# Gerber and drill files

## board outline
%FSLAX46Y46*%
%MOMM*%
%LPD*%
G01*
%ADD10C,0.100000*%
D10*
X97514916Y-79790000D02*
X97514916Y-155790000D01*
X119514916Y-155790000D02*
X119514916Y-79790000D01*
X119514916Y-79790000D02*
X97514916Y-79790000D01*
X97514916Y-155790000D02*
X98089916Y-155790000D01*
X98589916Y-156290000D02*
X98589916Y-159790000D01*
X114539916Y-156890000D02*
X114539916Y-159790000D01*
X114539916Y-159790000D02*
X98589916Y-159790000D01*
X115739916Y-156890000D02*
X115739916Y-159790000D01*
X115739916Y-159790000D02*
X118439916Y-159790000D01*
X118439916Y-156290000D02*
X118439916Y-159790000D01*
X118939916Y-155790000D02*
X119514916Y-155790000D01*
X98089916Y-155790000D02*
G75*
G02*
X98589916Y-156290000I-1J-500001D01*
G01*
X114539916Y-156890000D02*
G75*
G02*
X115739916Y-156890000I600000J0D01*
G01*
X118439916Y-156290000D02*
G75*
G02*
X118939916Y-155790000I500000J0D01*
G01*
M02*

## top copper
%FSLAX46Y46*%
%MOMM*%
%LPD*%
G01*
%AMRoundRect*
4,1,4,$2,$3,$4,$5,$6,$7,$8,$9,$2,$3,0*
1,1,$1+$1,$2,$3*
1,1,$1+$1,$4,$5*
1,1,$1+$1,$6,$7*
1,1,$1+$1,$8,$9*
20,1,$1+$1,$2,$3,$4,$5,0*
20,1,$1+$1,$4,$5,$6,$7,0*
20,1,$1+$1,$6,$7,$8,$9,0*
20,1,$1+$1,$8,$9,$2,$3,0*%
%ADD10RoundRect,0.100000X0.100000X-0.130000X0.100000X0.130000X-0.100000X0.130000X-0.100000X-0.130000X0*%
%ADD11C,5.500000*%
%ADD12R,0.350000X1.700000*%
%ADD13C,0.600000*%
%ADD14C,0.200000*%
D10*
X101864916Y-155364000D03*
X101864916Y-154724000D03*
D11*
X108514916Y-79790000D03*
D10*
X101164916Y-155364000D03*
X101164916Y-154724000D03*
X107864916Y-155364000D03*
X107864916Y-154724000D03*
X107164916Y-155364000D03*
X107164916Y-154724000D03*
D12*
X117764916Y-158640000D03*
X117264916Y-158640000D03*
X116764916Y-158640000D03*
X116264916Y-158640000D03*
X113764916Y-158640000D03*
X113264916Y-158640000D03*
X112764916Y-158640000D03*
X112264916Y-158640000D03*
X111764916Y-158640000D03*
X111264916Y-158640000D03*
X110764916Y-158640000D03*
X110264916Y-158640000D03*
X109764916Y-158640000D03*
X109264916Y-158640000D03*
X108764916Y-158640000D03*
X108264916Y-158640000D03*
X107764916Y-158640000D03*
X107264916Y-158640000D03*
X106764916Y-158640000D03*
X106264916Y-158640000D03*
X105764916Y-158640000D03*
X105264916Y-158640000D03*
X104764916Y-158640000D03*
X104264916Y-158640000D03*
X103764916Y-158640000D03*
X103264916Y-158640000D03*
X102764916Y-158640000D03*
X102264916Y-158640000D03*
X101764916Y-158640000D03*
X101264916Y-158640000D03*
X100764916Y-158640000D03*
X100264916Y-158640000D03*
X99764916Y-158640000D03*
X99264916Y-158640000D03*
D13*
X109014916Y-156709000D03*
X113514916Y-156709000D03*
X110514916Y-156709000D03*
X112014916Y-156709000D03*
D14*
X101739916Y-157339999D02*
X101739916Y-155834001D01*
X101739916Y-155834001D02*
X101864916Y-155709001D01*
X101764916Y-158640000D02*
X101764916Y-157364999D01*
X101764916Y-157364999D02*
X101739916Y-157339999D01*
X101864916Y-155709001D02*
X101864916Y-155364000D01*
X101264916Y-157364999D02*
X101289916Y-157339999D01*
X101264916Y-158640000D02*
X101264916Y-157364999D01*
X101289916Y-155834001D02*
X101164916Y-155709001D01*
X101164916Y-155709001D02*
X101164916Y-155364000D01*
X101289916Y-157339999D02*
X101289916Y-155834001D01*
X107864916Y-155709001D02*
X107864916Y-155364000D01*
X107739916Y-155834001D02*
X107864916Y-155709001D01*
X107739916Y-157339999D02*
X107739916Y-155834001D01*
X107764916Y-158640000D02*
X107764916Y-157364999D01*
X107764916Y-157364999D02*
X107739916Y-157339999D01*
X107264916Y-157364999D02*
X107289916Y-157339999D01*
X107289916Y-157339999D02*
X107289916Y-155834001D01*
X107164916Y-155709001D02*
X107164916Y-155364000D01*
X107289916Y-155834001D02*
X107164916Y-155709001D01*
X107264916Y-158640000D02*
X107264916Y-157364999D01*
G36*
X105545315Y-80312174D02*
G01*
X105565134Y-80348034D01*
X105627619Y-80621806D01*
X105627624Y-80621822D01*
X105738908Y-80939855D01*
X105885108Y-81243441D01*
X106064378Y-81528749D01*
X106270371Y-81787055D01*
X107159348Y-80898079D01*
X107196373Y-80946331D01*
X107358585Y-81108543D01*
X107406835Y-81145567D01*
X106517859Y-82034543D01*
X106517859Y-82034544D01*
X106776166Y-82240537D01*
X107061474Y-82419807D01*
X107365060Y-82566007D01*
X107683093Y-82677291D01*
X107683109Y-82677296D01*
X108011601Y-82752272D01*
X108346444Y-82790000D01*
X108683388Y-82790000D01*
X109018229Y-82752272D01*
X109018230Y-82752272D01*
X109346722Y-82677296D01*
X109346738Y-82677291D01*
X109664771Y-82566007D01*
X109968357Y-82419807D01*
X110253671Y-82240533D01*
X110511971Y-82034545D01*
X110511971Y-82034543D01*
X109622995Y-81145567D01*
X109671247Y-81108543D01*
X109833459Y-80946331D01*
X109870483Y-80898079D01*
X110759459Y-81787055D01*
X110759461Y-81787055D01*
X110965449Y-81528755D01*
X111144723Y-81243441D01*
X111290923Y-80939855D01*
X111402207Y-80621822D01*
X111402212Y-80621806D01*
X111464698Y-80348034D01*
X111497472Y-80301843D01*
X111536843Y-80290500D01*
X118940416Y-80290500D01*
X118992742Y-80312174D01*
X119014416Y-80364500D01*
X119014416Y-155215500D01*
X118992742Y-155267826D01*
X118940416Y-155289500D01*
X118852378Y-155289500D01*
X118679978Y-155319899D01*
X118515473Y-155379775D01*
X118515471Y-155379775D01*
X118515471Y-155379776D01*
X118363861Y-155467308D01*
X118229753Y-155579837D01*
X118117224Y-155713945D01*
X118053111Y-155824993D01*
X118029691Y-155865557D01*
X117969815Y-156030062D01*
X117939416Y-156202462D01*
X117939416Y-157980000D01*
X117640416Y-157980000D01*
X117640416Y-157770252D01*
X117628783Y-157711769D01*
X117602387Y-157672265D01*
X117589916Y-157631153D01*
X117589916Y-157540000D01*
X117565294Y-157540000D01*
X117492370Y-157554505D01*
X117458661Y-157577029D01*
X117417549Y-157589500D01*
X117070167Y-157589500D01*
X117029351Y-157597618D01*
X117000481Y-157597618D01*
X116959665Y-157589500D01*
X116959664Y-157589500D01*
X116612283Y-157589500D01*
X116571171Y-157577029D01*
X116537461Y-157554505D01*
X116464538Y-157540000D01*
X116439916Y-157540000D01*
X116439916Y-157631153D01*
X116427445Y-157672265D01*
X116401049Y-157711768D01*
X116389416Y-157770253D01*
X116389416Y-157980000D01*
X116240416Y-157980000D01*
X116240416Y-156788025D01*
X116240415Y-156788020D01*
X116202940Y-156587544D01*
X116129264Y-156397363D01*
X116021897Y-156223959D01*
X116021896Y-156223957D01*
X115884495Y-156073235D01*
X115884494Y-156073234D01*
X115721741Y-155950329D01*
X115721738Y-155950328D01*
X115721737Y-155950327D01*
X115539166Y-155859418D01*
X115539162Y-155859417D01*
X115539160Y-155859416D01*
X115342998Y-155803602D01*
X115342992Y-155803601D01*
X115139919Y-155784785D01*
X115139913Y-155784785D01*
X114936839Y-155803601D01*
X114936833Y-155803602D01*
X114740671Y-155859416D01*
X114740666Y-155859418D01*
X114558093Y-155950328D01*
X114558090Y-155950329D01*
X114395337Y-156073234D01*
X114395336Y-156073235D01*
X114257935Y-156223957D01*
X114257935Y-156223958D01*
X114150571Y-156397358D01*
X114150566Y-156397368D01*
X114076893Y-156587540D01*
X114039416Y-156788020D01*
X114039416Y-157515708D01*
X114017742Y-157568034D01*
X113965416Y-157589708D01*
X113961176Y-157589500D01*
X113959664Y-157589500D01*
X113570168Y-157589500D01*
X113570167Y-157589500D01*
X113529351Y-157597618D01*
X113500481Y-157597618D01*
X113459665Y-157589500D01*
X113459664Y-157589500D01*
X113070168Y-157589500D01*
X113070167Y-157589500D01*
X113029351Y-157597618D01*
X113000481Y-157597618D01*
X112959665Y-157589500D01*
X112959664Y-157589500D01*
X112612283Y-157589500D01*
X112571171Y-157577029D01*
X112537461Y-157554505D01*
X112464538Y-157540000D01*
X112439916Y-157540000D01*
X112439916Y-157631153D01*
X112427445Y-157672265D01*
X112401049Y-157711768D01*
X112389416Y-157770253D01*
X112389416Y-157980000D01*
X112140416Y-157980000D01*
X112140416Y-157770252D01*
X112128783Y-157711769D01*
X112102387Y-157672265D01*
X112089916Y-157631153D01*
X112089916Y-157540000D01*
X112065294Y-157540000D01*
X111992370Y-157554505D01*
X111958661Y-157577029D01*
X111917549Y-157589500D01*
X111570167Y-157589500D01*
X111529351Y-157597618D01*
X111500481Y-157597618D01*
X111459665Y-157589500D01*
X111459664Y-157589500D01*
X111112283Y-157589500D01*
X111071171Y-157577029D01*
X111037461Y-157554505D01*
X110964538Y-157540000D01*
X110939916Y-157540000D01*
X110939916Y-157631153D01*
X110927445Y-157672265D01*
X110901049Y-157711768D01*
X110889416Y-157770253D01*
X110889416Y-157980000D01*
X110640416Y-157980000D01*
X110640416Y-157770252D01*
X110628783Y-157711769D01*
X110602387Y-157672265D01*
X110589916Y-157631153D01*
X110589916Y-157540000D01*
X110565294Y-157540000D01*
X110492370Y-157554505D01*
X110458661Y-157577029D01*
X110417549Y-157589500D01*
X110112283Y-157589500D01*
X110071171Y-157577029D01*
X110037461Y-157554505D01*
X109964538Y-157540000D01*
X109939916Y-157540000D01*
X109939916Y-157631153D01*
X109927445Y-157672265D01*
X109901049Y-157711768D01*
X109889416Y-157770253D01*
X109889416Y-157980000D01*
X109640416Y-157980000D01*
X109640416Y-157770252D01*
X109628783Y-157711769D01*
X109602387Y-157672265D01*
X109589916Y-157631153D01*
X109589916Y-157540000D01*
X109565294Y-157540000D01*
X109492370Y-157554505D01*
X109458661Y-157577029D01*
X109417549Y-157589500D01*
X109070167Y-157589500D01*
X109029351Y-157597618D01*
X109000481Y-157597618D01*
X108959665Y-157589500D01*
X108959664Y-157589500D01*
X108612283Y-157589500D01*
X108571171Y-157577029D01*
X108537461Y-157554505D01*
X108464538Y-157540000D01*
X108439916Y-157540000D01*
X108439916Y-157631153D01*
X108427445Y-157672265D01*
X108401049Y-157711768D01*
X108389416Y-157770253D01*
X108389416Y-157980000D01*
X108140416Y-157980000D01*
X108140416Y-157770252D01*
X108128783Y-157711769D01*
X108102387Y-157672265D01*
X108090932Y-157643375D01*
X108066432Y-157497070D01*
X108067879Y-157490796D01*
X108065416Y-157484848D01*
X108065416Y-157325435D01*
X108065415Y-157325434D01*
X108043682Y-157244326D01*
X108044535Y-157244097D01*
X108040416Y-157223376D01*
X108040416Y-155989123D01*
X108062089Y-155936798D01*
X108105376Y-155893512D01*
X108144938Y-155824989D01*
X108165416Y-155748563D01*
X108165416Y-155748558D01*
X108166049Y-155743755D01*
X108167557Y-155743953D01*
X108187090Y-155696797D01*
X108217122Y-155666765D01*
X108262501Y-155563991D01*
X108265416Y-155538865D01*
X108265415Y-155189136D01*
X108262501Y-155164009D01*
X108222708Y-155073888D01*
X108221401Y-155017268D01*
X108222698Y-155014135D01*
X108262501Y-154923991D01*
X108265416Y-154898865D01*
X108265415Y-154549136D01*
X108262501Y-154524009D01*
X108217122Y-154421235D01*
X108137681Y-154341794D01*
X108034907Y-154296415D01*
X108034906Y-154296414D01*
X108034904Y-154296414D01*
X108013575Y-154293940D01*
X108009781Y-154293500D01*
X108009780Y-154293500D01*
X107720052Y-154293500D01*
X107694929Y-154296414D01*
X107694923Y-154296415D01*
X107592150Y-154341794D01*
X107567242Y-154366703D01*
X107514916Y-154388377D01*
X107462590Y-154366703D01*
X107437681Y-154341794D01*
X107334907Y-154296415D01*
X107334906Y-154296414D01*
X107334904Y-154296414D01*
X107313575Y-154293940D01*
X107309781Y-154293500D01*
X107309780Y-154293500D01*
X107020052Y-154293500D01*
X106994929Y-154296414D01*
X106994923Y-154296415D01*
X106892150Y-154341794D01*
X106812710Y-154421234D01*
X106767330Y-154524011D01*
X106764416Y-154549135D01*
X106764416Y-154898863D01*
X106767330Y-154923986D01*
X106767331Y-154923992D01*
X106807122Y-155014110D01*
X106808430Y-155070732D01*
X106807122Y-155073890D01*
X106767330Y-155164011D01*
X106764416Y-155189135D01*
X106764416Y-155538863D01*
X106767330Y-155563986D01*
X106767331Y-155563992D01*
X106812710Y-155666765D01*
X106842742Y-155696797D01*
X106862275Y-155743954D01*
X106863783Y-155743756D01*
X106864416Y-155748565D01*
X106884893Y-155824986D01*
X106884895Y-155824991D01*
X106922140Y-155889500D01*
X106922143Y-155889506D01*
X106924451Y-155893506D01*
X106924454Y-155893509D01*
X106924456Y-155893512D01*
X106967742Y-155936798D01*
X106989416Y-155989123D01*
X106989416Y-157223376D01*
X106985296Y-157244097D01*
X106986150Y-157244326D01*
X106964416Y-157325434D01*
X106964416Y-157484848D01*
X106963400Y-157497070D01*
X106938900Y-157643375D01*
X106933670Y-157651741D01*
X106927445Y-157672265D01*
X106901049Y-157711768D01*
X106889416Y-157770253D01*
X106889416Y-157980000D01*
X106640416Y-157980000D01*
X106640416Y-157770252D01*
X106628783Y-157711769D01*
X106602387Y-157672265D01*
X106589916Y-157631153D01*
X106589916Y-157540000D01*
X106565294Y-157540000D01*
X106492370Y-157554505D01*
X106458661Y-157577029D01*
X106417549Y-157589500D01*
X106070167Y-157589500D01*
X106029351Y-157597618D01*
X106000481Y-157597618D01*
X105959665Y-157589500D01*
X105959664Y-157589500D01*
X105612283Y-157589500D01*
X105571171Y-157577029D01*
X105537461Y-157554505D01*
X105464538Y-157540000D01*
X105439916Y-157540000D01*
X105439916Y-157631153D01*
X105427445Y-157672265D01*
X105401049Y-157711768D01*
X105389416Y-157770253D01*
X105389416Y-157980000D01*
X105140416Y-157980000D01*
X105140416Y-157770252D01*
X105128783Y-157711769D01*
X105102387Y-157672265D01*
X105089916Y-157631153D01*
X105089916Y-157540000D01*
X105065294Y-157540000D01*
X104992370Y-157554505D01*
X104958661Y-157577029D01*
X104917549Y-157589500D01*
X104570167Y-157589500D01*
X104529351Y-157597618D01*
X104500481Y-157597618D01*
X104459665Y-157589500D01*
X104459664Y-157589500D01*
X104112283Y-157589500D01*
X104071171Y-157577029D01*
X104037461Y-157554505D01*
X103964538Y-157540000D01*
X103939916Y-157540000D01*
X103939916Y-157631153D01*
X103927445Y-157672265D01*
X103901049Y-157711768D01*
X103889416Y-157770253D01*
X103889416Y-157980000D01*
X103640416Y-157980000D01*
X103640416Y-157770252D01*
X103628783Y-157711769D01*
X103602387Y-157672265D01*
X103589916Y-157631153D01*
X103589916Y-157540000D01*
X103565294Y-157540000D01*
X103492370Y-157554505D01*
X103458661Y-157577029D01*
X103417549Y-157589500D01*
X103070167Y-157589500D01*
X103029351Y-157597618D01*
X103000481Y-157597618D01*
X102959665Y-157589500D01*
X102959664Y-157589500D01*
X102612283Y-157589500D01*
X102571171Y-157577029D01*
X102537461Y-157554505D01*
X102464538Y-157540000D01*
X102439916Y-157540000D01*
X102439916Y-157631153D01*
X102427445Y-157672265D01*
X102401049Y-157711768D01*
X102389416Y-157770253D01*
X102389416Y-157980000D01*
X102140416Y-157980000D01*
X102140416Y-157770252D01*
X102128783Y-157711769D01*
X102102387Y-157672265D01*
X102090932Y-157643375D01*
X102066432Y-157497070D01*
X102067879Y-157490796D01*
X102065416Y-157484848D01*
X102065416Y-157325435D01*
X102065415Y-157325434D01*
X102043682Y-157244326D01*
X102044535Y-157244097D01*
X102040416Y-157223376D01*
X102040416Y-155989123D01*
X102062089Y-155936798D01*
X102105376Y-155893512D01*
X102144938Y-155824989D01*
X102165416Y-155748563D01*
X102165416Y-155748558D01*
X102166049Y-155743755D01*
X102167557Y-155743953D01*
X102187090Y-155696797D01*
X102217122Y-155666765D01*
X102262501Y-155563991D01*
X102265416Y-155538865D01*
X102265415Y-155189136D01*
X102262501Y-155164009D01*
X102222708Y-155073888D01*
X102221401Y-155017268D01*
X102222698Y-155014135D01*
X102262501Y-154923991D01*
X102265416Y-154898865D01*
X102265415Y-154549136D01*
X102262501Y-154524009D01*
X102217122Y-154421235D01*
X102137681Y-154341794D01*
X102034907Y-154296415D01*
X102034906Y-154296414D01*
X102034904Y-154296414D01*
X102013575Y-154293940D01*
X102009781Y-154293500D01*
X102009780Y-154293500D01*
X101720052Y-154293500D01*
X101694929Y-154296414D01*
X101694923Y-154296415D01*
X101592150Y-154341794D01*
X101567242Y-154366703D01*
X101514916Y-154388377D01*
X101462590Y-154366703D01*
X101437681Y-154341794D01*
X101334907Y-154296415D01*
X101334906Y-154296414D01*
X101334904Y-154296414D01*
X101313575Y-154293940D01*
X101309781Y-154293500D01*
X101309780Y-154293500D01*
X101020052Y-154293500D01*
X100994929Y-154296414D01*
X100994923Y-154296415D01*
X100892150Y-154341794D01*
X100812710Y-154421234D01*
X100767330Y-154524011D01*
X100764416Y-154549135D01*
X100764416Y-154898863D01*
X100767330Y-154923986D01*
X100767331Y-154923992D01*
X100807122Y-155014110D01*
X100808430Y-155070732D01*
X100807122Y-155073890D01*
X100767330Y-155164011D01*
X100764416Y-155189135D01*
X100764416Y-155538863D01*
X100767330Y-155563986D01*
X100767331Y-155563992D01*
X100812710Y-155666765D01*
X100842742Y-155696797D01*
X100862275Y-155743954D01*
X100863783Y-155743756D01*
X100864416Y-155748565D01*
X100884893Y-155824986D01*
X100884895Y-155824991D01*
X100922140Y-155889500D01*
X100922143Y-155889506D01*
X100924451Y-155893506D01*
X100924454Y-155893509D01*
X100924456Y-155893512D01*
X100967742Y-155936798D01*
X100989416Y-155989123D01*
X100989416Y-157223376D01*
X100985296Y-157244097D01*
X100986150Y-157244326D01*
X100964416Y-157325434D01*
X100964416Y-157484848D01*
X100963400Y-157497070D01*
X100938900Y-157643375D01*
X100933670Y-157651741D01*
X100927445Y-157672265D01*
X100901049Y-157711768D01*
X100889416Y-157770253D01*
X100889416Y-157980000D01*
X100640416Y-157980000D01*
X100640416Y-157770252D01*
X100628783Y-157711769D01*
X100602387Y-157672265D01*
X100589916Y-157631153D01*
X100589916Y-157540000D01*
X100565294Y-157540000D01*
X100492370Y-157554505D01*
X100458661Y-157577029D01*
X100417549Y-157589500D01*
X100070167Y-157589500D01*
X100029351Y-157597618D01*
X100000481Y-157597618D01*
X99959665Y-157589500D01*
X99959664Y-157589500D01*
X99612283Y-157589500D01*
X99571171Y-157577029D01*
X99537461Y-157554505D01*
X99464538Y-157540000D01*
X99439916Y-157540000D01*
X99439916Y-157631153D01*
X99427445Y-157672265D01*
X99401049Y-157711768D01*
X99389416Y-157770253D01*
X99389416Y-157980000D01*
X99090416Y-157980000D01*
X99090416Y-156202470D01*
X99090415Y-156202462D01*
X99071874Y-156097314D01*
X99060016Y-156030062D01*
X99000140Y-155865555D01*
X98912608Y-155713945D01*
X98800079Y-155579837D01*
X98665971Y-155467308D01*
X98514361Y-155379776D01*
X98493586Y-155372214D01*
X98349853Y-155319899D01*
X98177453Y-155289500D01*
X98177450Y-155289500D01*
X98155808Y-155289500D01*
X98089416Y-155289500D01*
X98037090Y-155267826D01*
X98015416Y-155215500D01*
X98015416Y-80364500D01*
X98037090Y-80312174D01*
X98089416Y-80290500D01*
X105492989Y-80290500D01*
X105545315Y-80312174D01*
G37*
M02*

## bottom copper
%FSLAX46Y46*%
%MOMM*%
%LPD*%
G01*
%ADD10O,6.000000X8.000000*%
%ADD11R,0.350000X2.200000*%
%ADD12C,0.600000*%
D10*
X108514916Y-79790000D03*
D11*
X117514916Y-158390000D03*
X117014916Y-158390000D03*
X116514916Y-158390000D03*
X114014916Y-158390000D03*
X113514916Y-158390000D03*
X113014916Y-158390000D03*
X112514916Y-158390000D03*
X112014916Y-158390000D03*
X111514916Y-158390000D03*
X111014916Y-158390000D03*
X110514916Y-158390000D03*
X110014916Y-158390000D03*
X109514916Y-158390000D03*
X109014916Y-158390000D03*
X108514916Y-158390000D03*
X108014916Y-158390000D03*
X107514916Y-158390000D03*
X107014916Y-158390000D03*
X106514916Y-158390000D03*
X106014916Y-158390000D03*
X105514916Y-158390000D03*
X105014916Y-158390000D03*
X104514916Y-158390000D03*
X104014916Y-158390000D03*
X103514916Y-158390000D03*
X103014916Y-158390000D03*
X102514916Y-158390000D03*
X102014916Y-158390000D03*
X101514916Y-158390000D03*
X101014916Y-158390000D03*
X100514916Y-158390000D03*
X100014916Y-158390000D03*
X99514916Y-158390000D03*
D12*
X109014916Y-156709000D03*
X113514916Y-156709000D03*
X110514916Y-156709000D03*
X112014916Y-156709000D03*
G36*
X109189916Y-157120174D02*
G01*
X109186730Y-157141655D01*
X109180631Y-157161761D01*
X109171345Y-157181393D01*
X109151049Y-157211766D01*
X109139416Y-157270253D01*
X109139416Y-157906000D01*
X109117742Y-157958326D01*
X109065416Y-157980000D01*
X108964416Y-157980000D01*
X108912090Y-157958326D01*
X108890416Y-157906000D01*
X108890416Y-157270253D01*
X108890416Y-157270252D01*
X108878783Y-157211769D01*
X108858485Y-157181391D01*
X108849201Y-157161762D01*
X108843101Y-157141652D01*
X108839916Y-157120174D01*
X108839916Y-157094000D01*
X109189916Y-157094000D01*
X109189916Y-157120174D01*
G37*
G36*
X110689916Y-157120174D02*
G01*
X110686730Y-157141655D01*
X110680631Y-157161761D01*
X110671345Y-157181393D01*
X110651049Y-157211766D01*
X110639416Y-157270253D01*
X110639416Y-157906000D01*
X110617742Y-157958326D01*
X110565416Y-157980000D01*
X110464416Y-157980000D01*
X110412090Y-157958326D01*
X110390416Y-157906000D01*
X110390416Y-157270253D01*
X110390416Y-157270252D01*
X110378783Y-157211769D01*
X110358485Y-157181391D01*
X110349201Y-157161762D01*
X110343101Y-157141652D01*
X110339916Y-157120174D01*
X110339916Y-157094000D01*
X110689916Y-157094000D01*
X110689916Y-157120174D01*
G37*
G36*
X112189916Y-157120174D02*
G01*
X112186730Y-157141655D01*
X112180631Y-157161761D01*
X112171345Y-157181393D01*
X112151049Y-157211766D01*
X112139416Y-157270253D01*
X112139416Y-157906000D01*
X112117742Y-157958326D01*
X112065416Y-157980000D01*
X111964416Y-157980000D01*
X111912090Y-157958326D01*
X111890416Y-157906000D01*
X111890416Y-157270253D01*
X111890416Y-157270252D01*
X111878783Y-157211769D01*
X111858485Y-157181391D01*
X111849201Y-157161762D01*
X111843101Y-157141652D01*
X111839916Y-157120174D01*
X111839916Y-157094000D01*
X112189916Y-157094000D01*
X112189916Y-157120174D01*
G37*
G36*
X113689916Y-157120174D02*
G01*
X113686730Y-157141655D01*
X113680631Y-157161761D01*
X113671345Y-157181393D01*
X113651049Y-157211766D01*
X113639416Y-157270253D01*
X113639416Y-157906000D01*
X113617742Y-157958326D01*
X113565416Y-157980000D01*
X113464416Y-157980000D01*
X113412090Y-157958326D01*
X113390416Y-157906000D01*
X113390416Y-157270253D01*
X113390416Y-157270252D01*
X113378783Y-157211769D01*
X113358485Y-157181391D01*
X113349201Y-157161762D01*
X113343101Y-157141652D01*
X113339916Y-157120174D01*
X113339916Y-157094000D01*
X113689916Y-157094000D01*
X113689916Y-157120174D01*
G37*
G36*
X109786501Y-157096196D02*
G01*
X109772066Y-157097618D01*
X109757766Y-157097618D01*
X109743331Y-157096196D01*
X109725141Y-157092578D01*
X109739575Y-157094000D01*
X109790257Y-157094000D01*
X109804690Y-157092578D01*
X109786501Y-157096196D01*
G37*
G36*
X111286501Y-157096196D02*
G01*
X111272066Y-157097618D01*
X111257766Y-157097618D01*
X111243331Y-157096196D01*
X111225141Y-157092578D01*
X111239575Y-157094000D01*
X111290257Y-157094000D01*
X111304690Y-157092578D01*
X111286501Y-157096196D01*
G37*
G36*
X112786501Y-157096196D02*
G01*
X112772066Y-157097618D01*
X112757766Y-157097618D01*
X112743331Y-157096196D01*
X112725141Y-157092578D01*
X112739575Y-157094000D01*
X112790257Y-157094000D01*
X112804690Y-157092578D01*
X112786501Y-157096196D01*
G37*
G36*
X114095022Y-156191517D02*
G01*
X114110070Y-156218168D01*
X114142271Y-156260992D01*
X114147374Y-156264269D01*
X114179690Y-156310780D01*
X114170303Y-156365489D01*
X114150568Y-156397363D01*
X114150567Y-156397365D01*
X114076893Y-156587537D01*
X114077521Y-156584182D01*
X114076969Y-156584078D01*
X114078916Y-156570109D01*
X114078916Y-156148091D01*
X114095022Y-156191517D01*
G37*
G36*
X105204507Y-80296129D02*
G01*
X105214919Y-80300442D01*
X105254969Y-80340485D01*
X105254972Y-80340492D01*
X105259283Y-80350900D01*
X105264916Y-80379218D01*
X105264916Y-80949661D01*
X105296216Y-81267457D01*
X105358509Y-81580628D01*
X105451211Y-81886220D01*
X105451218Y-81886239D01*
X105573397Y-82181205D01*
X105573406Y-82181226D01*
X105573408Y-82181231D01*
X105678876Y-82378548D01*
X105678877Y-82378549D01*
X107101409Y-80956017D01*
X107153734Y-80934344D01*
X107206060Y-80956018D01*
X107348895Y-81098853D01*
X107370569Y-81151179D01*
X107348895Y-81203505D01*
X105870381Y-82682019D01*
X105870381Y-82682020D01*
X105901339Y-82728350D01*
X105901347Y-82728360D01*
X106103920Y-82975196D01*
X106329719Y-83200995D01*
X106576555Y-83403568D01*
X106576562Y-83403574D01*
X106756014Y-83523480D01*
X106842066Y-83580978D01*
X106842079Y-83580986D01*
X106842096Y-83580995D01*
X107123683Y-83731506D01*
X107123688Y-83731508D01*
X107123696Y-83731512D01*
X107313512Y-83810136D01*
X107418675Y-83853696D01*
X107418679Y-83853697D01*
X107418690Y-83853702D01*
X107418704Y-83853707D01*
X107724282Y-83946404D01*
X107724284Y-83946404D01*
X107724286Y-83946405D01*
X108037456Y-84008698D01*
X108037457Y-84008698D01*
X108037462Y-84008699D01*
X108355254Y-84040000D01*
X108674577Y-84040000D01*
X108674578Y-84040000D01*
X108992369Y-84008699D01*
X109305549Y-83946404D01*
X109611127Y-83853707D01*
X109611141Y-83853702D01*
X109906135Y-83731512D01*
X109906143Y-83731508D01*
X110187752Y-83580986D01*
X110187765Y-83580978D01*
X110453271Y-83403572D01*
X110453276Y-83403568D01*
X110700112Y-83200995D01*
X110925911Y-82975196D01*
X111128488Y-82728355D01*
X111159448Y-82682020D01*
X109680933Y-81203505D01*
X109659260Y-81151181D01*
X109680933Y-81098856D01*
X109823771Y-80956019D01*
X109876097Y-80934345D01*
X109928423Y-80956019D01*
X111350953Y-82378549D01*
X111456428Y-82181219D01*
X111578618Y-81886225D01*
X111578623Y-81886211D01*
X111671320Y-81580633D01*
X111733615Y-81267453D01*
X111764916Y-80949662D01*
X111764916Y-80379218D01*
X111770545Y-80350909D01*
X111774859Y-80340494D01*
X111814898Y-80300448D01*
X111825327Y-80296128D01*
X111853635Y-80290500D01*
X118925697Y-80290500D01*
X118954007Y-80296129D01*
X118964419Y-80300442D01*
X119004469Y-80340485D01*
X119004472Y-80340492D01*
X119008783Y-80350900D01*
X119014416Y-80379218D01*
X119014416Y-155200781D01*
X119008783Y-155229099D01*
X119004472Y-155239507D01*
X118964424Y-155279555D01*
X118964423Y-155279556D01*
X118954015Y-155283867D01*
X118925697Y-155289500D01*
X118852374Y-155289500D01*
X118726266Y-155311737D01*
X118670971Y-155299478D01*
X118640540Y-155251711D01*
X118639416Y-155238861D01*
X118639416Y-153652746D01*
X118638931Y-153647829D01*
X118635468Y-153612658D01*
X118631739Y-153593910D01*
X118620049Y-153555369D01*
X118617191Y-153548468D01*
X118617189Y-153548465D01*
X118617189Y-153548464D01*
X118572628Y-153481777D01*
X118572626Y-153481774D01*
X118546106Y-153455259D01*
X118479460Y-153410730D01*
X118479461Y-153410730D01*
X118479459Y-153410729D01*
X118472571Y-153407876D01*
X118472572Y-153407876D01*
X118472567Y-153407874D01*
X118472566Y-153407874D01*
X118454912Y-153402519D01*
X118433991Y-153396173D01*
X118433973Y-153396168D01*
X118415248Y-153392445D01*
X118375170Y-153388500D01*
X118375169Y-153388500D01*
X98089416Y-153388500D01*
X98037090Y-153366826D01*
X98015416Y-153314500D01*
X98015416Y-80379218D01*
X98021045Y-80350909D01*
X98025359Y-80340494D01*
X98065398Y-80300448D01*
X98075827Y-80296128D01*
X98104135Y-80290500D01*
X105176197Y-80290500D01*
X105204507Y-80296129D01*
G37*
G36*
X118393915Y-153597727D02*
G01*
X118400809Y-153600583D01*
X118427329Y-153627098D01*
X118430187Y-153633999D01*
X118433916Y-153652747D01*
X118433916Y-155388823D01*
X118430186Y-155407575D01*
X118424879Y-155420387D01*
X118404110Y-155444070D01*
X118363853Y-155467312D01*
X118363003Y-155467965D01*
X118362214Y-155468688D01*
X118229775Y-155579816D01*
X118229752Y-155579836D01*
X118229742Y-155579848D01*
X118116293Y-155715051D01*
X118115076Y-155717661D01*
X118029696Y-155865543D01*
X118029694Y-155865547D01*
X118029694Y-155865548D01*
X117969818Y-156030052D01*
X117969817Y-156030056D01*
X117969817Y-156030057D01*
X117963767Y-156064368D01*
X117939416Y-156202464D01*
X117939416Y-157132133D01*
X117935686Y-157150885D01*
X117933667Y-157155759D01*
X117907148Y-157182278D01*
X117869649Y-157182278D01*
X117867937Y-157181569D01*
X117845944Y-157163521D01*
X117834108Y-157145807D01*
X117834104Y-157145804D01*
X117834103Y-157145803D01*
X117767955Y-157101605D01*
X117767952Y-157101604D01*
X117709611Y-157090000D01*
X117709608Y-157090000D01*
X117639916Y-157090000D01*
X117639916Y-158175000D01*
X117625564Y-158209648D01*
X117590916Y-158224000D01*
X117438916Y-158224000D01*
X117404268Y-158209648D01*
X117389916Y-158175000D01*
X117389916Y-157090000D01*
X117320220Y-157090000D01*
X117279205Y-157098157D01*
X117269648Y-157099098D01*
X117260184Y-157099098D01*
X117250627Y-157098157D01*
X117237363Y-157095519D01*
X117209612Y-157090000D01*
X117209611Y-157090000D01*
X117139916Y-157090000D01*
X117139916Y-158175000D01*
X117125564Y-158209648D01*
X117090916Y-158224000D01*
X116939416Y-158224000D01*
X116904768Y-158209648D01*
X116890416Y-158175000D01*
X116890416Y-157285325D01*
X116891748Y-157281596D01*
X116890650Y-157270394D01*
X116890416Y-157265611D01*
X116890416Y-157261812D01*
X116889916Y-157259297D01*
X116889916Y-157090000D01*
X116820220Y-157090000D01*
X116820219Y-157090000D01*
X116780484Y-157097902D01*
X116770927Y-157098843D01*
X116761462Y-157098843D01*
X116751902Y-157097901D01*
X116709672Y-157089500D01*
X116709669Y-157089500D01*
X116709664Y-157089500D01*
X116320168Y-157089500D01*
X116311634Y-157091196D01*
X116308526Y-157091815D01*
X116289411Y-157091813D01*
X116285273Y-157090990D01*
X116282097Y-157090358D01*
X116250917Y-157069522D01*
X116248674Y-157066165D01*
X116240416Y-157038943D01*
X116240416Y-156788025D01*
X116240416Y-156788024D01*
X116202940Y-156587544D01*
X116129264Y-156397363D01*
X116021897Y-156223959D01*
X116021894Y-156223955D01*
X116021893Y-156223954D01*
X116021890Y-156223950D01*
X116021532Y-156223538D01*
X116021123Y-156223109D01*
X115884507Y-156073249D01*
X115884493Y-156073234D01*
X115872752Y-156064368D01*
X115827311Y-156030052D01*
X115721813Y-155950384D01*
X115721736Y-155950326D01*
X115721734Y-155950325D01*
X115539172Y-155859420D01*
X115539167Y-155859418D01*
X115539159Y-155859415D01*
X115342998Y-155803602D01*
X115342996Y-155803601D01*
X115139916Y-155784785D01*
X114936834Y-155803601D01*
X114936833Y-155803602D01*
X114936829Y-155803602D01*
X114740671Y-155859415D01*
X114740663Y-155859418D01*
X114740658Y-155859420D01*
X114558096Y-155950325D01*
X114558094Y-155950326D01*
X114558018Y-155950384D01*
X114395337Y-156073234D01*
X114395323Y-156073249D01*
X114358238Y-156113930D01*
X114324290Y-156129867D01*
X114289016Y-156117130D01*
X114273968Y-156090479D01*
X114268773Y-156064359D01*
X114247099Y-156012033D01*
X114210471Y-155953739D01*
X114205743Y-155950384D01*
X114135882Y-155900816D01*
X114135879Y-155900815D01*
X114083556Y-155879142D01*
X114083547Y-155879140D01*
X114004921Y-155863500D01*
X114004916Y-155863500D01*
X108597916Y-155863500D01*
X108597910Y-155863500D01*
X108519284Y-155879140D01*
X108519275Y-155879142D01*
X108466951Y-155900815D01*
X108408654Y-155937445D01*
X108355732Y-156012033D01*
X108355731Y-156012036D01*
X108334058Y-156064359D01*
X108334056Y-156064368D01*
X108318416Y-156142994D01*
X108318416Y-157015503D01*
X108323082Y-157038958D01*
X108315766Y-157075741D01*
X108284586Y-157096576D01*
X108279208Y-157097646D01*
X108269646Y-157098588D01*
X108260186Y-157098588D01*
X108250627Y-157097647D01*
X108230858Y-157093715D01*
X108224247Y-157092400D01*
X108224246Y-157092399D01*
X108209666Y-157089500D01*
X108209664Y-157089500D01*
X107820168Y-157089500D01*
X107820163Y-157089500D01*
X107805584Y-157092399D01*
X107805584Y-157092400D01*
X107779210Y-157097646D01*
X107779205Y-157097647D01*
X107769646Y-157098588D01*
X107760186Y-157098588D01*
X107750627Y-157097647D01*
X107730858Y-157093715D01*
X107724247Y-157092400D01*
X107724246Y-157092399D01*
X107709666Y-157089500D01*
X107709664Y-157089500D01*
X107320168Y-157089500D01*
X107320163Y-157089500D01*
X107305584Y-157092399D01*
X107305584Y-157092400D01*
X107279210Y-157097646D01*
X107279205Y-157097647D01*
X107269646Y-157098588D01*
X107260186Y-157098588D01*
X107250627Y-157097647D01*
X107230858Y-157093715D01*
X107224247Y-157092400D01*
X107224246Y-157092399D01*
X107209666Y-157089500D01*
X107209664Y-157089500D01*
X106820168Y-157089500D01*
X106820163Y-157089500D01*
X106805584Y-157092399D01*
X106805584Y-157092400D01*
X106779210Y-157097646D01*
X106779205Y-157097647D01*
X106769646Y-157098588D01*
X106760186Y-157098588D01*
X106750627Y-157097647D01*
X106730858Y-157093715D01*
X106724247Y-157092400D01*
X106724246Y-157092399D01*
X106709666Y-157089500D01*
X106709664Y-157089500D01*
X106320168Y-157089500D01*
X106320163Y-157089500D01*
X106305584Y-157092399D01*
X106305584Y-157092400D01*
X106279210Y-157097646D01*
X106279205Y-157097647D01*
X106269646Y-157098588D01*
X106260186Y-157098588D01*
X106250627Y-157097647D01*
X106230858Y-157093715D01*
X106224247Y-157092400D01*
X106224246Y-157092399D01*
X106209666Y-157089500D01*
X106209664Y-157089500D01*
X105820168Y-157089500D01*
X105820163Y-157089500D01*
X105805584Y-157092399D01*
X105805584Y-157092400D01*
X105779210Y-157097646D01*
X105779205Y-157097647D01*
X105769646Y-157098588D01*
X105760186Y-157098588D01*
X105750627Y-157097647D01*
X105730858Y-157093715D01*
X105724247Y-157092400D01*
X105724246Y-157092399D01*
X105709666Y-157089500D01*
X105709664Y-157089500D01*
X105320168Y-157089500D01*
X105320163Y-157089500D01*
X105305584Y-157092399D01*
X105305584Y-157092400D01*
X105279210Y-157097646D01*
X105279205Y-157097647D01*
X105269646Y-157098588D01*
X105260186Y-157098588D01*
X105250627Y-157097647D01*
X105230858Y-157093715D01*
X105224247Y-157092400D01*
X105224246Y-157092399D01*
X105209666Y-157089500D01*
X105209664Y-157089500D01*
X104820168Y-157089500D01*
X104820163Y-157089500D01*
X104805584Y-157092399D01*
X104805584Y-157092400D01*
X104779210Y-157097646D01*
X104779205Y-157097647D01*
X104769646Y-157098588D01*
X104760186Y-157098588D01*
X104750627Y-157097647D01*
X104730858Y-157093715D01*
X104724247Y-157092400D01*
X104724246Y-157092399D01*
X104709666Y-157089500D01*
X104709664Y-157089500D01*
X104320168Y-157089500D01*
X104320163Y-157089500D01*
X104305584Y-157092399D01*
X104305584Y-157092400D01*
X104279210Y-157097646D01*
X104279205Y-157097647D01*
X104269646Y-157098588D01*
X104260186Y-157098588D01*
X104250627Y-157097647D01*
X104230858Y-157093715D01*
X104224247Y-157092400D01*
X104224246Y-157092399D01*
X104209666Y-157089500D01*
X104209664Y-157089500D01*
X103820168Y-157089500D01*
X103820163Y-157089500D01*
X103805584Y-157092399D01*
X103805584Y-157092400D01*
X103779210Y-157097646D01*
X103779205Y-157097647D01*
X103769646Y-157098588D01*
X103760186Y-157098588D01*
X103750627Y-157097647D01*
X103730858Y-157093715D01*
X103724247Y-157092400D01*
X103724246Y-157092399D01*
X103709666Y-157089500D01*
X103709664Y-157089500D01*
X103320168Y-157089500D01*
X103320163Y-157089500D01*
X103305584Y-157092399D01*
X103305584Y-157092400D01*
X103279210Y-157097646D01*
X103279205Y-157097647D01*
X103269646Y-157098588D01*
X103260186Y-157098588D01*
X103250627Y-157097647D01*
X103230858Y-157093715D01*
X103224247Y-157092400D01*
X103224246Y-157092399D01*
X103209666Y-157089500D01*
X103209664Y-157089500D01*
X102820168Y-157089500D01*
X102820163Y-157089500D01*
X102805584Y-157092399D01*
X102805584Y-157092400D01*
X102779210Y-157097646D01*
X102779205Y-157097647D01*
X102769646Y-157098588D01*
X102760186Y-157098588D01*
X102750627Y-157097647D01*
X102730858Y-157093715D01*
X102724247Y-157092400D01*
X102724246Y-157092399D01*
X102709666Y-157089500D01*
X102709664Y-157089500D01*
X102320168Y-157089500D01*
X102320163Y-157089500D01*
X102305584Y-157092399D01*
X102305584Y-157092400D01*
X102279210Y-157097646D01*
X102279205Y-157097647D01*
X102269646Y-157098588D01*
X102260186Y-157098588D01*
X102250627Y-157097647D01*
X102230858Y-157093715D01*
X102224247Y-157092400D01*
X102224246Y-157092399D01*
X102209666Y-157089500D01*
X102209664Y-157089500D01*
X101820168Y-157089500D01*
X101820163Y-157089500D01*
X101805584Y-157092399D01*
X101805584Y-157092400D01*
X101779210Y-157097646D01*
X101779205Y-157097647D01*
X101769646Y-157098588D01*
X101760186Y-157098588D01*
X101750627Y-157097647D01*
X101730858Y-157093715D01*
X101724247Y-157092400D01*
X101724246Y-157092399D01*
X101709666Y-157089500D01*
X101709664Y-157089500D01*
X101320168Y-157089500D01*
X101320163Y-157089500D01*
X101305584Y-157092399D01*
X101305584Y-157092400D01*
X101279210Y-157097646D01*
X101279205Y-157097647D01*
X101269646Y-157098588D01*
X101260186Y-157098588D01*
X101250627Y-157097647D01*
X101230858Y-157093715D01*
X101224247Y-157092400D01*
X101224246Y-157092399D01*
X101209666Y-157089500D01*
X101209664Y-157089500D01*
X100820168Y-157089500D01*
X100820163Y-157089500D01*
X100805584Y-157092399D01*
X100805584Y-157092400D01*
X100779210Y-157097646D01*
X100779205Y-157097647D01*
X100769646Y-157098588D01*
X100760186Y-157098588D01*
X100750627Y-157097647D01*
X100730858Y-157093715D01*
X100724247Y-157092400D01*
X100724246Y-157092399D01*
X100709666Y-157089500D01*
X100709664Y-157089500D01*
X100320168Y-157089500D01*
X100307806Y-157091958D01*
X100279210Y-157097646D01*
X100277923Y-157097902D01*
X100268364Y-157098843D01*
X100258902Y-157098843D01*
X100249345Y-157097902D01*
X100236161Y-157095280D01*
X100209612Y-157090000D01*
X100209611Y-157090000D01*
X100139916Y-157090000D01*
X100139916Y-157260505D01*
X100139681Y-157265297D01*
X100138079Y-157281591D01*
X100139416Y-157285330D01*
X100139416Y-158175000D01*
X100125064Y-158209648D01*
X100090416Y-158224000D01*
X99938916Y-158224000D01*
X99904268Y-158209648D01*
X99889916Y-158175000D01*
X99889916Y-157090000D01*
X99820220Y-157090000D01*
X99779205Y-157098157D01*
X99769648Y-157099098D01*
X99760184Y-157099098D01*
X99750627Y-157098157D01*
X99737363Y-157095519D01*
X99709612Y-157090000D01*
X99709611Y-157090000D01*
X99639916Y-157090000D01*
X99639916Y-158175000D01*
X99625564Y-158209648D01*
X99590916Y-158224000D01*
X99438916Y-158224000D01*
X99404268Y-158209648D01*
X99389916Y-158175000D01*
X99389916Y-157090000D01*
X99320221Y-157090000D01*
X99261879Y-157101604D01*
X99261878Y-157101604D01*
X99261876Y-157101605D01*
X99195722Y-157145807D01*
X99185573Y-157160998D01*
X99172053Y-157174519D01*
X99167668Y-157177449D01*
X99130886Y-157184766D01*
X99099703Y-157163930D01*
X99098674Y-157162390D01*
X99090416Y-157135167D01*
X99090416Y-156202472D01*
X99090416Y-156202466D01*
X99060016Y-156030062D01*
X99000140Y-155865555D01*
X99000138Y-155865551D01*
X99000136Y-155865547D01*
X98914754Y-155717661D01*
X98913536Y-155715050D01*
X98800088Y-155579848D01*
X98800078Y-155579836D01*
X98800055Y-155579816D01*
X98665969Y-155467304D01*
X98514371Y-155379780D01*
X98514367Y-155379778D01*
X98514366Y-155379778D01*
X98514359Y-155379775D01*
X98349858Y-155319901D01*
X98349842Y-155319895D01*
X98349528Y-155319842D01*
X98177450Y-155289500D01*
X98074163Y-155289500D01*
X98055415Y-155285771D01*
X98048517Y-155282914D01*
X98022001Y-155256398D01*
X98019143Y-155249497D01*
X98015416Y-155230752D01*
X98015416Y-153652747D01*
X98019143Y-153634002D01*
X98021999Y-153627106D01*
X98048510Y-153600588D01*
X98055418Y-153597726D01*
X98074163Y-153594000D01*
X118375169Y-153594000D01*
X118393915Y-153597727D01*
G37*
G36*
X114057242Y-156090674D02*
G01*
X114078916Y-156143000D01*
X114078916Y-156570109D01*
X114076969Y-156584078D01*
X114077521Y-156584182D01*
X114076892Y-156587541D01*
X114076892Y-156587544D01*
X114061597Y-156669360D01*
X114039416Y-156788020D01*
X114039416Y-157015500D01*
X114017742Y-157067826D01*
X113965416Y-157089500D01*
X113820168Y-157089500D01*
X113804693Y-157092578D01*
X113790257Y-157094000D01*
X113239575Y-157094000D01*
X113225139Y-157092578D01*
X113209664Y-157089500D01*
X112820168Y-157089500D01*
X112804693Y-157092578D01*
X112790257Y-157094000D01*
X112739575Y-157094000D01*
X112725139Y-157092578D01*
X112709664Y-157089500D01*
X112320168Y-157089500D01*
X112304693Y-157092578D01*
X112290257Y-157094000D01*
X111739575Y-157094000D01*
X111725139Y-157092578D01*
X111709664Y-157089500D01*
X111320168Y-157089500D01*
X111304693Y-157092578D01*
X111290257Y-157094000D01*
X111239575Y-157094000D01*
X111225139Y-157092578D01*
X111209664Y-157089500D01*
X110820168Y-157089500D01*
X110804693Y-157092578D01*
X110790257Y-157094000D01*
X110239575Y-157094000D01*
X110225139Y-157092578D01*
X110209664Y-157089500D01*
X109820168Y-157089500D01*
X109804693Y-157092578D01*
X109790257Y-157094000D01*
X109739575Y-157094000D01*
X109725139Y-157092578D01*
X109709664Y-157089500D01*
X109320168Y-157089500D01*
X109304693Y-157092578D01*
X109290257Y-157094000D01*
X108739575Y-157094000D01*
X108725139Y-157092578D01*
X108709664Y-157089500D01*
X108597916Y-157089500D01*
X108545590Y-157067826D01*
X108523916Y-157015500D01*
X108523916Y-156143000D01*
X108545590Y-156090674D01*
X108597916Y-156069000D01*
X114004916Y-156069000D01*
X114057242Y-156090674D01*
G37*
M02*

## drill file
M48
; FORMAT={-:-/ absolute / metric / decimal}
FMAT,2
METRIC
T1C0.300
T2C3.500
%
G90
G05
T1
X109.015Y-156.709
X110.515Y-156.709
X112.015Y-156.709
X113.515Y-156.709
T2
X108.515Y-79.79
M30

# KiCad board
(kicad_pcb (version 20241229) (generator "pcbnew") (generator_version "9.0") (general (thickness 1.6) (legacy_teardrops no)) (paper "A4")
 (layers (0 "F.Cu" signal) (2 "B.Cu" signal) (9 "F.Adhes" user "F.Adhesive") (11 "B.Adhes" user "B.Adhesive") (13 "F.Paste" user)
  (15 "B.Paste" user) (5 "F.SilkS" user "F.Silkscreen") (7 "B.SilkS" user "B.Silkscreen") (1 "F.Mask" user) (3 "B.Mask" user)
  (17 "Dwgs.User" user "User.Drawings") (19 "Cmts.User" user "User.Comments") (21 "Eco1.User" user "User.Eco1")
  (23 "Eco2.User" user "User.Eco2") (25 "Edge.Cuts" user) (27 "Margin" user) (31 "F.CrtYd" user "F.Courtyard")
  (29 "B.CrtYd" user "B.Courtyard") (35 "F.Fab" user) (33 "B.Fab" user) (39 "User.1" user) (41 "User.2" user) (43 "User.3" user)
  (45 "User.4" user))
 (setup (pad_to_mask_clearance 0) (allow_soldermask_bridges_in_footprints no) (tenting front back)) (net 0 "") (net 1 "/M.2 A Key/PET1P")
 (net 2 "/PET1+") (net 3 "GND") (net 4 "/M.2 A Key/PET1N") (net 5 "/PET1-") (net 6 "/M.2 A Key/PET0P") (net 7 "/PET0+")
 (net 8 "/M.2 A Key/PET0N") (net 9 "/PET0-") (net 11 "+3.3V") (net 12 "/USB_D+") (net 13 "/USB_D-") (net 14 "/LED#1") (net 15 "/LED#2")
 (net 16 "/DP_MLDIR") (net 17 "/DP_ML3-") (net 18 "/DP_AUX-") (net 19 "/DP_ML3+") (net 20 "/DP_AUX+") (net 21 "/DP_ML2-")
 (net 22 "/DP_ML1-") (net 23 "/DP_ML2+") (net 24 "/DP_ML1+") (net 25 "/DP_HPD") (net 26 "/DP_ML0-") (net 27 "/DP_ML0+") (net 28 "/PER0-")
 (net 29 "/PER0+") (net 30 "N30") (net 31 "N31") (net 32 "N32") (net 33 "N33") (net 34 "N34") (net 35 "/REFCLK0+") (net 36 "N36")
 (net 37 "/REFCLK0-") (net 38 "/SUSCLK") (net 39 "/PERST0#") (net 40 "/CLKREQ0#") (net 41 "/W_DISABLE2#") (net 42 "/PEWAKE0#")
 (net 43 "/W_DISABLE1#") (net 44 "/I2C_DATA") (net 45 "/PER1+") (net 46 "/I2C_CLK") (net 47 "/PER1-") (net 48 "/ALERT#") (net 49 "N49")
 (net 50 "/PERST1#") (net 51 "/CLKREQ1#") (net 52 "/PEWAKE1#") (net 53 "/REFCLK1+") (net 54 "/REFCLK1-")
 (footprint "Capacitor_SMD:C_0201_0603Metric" (layer "F.Cu") (at 101.864916 155.044 90)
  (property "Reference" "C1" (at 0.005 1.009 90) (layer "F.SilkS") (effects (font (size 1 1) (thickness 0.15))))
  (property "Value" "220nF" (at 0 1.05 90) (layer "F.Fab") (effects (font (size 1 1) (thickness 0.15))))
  (pad "" smd roundrect (at -0.345 0 90) (size 0.318 0.36) (layers "F.Paste") (roundrect_rratio 0.25))
  (pad "" smd roundrect (at 0.345 0 90) (size 0.318 0.36) (layers "F.Paste") (roundrect_rratio 0.25))
  (pad "1" smd roundrect (at -0.32 0 90) (size 0.46 0.4) (layers "F.Cu" "F.Mask") (roundrect_rratio 0.25) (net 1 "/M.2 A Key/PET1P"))
  (pad "2" smd roundrect (at 0.32 0 90) (size 0.46 0.4) (layers "F.Cu" "F.Mask") (roundrect_rratio 0.25) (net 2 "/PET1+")))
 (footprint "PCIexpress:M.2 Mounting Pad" (layer "F.Cu") (at 108.514916 129.79)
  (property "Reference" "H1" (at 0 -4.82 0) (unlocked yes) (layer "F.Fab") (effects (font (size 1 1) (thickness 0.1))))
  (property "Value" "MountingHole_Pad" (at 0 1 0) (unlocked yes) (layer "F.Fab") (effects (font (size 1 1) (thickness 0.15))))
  (pad "1" thru_hole circle (at 0 -50) (size 5.5 5.5) (drill 3.5) (layers "*.Cu" "*.Mask") (remove_unused_layers no) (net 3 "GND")
   (padstack (mode front_inner_back)
    (layer "Inner" (shape circle) (size 5.5 5.5) (zone_connect -1))
    (layer "B.Cu" (shape oval) (size 6 8) (thermal_bridge_angle 45) (zone_connect -1)))))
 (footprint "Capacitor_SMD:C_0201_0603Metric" (layer "F.Cu") (at 101.164916 155.044 90)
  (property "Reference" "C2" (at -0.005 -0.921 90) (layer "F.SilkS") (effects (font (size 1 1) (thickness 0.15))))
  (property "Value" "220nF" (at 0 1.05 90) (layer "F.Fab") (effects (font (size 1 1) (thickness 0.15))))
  (pad "" smd roundrect (at -0.345 0 90) (size 0.318 0.36) (layers "F.Paste") (roundrect_rratio 0.25))
  (pad "" smd roundrect (at 0.345 0 90) (size 0.318 0.36) (layers "F.Paste") (roundrect_rratio 0.25))
  (pad "1" smd roundrect (at -0.32 0 90) (size 0.46 0.4) (layers "F.Cu" "F.Mask") (roundrect_rratio 0.25) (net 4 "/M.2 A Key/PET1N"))
  (pad "2" smd roundrect (at 0.32 0 90) (size 0.46 0.4) (layers "F.Cu" "F.Mask") (roundrect_rratio 0.25) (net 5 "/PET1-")))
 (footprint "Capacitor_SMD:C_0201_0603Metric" (layer "F.Cu") (at 107.864916 155.044 90)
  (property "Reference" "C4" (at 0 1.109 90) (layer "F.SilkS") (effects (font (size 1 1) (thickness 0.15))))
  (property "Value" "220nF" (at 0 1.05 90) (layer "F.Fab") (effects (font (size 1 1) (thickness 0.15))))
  (pad "" smd roundrect (at -0.345 0 90) (size 0.318 0.36) (layers "F.Paste") (roundrect_rratio 0.25))
  (pad "" smd roundrect (at 0.345 0 90) (size 0.318 0.36) (layers "F.Paste") (roundrect_rratio 0.25))
  (pad "1" smd roundrect (at -0.32 0 90) (size 0.46 0.4) (layers "F.Cu" "F.Mask") (roundrect_rratio 0.25) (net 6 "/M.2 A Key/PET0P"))
  (pad "2" smd roundrect (at 0.32 0 90) (size 0.46 0.4) (layers "F.Cu" "F.Mask") (roundrect_rratio 0.25) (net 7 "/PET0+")))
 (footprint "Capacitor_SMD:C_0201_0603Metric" (layer "F.Cu") (at 107.164916 155.044 90)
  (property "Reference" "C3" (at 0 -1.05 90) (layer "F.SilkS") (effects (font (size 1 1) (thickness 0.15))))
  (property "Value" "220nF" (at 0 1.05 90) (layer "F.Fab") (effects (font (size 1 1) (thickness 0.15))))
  (pad "" smd roundrect (at -0.345 0 90) (size 0.318 0.36) (layers "F.Paste") (roundrect_rratio 0.25))
  (pad "" smd roundrect (at 0.345 0 90) (size 0.318 0.36) (layers "F.Paste") (roundrect_rratio 0.25))
  (pad "1" smd roundrect (at -0.32 0 90) (size 0.46 0.4) (layers "F.Cu" "F.Mask") (roundrect_rratio 0.25) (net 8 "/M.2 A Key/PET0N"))
  (pad "2" smd roundrect (at 0.32 0 90) (size 0.46 0.4) (layers "F.Cu" "F.Mask") (roundrect_rratio 0.25) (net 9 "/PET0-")))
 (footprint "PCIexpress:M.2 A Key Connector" (layer "F.Cu") (at 108.514916 158.68)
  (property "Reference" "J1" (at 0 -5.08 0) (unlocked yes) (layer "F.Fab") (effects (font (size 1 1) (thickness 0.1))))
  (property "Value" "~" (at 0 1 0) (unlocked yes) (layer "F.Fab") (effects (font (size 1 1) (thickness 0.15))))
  (fp_line (start -11 -2.89) (end -10.425 -2.89) (stroke (width 0.1) (type default)) (layer "Edge.Cuts") (net 10))
  (fp_line (start -9.925 -2.39) (end -9.925 1.11) (stroke (width 0.1) (type default)) (layer "Edge.Cuts") (net 10))
  (fp_line (start 6.025 -1.79) (end 6.025 1.11) (stroke (width 0.1) (type default)) (layer "Edge.Cuts") (net 10))
  (fp_line (start 6.025 1.11) (end -9.925 1.11) (stroke (width 0.1) (type default)) (layer "Edge.Cuts") (net 10))
  (fp_line (start 7.225 -1.79) (end 7.225 1.11) (stroke (width 0.1) (type default)) (layer "Edge.Cuts") (net 10))
  (fp_line (start 7.225 1.11) (end 9.925 1.11) (stroke (width 0.1) (type default)) (layer "Edge.Cuts") (net 10))
  (fp_line (start 9.925 -2.39) (end 9.925 1.11) (stroke (width 0.1) (type default)) (layer "Edge.Cuts") (net 10))
  (fp_line (start 10.425 -2.89) (end 11 -2.89) (stroke (width 0.1) (type default)) (layer "Edge.Cuts") (net 10))
  (fp_arc (start -10.425 -2.89) (mid -10.071447 -2.743553) (end -9.925 -2.39) (stroke (width 0.1) (type default)) (layer "Edge.Cuts")
   (net 10))
  (fp_arc (start 6.025 -1.79) (mid 6.625 -2.39) (end 7.225 -1.79) (stroke (width 0.1) (type default)) (layer "Edge.Cuts") (net 10))
  (fp_arc (start 9.925 -2.39) (mid 10.071447 -2.743553) (end 10.425 -2.89) (stroke (width 0.1) (type default)) (layer "Edge.Cuts") (net 10))
  (pad "1" smd rect (at 9.25 -0.04 180) (size 0.35 1.7) (layers "F.Cu") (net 3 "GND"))
  (pad "2" smd rect (at 9 -0.29 180) (size 0.35 2.2) (layers "B.Cu") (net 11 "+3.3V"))
  (pad "3" smd rect (at 8.75 -0.04 180) (size 0.35 1.7) (layers "F.Cu") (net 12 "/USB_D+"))
  (pad "4" smd rect (at 8.5 -0.29 180) (size 0.35 2.2) (layers "B.Cu") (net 11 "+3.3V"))
  (pad "5" smd rect (at 8.25 -0.04 180) (size 0.35 1.7) (layers "F.Cu") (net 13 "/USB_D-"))
  (pad "6" smd rect (at 8 -0.29 180) (size 0.35 2.2) (layers "B.Cu") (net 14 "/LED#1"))
  (pad "7" smd rect (at 7.75 -0.04 180) (size 0.35 1.7) (layers "F.Cu") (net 3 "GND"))
  (pad "16" smd rect (at 5.5 -0.29 180) (size 0.35 2.2) (layers "B.Cu") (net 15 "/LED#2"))
  (pad "17" smd rect (at 5.25 -0.04 180) (size 0.35 1.7) (layers "F.Cu") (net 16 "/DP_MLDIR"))
  (pad "18" smd rect (at 5 -0.29 180) (size 0.35 2.2) (layers "B.Cu") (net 3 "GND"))
  (pad "19" smd rect (at 4.75 -0.04 180) (size 0.35 1.7) (layers "F.Cu") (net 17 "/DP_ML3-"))
  (pad "20" smd rect (at 4.5 -0.29 180) (size 0.35 2.2) (layers "B.Cu") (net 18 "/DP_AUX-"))
  (pad "21" smd rect (at 4.25 -0.04 180) (size 0.35 1.7) (layers "F.Cu") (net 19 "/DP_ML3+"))
  (pad "22" smd rect (at 4 -0.29 180) (size 0.35 2.2) (layers "B.Cu") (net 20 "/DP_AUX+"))
  (pad "23" smd rect (at 3.75 -0.04 180) (size 0.35 1.7) (layers "F.Cu") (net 3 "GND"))
  (pad "24" smd rect (at 3.5 -0.29 180) (size 0.35 2.2) (layers "B.Cu") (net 3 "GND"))
  (pad "25" smd rect (at 3.25 -0.04 180) (size 0.35 1.7) (layers "F.Cu") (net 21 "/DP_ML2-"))
  (pad "26" smd rect (at 3 -0.29 180) (size 0.35 2.2) (layers "B.Cu") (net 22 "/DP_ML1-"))
  (pad "27" smd rect (at 2.75 -0.04 180) (size 0.35 1.7) (layers "F.Cu") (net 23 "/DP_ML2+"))
  (pad "28" smd rect (at 2.5 -0.29 180) (size 0.35 2.2) (layers "B.Cu") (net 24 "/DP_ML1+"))
  (pad "29" smd rect (at 2.25 -0.04 180) (size 0.35 1.7) (layers "F.Cu") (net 3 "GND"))
  (pad "30" smd rect (at 2 -0.29 180) (size 0.35 2.2) (layers "B.Cu") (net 3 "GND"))
  (pad "31" smd rect (at 1.75 -0.04 180) (size 0.35 1.7) (layers "F.Cu") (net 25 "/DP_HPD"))
  (pad "32" smd rect (at 1.5 -0.29 180) (size 0.35 2.2) (layers "B.Cu") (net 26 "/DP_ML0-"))
  (pad "33" smd rect (at 1.25 -0.04 180) (size 0.35 1.7) (layers "F.Cu") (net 3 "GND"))
  (pad "34" smd rect (at 1 -0.29 180) (size 0.35 2.2) (layers "B.Cu") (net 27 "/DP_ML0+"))
  (pad "35" smd rect (at 0.75 -0.04 180) (size 0.35 1.7) (layers "F.Cu") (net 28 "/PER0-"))
  (pad "36" smd rect (at 0.5 -0.29 180) (size 0.35 2.2) (layers "B.Cu") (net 3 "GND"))
  (pad "37" smd rect (at 0.25 -0.04 180) (size 0.35 1.7) (layers "F.Cu") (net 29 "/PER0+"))
  (pad "38" smd rect (at 0 -0.29 180) (size 0.35 2.2) (layers "B.Cu") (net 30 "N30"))
  (pad "39" smd rect (at -0.25 -0.04 180) (size 0.35 1.7) (layers "F.Cu") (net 3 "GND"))
  (pad "40" smd rect (at -0.5 -0.29 180) (size 0.35 2.2) (layers "B.Cu") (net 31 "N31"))
  (pad "41" smd rect (at -0.75 -0.04 180) (size 0.35 1.7) (layers "F.Cu") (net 6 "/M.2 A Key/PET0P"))
  (pad "42" smd rect (at -1 -0.29 180) (size 0.35 2.2) (layers "B.Cu") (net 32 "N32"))
  (pad "43" smd rect (at -1.25 -0.04 180) (size 0.35 1.7) (layers "F.Cu") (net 8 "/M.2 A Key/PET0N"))
  (pad "44" smd rect (at -1.5 -0.29 180) (size 0.35 2.2) (layers "B.Cu") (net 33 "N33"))
  (pad "45" smd rect (at -1.75 -0.04 180) (size 0.35 1.7) (layers "F.Cu") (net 3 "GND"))
  (pad "46" smd rect (at -2 -0.29 180) (size 0.35 2.2) (layers "B.Cu") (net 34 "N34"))
  (pad "47" smd rect (at -2.25 -0.04 180) (size 0.35 1.7) (layers "F.Cu") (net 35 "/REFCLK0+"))
  (pad "48" smd rect (at -2.5 -0.29 180) (size 0.35 2.2) (layers "B.Cu") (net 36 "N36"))
  (pad "49" smd rect (at -2.75 -0.04 180) (size 0.35 1.7) (layers "F.Cu") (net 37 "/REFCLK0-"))
  (pad "50" smd rect (at -3 -0.29 180) (size 0.35 2.2) (layers "B.Cu") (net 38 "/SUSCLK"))
  (pad "51" smd rect (at -3.25 -0.04 180) (size 0.35 1.7) (layers "F.Cu") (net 3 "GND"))
  (pad "52" smd rect (at -3.5 -0.29 180) (size 0.35 2.2) (layers "B.Cu") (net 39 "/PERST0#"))
  (pad "53" smd rect (at -3.75 -0.04 180) (size 0.35 1.7) (layers "F.Cu") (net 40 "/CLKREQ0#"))
  (pad "54" smd rect (at -4 -0.29 180) (size 0.35 2.2) (layers "B.Cu") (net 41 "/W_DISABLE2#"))
  (pad "55" smd rect (at -4.25 -0.04 180) (size 0.35 1.7) (layers "F.Cu") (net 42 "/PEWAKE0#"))
  (pad "56" smd rect (at -4.5 -0.29 180) (size 0.35 2.2) (layers "B.Cu") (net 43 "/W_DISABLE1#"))
  (pad "57" smd rect (at -4.75 -0.04 180) (size 0.35 1.7) (layers "F.Cu") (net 3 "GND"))
  (pad "58" smd rect (at -5 -0.29 180) (size 0.35 2.2) (layers "B.Cu") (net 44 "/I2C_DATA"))
  (pad "59" smd rect (at -5.25 -0.04 180) (size 0.35 1.7) (layers "F.Cu") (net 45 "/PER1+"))
  (pad "60" smd rect (at -5.5 -0.29 180) (size 0.35 2.2) (layers "B.Cu") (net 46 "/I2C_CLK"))
  (pad "61" smd rect (at -5.75 -0.04 180) (size 0.35 1.7) (layers "F.Cu") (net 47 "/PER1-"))
  (pad "62" smd rect (at -6 -0.29 180) (size 0.35 2.2) (layers "B.Cu") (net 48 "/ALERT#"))
  (pad "63" smd rect (at -6.25 -0.04 180) (size 0.35 1.7) (layers "F.Cu") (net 3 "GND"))
  (pad "64" smd rect (at -6.5 -0.29 180) (size 0.35 2.2) (layers "B.Cu") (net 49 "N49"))
  (pad "65" smd rect (at -6.75 -0.04 180) (size 0.35 1.7) (layers "F.Cu") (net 1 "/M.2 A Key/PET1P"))
  (pad "66" smd rect (at -7 -0.29 180) (size 0.35 2.2) (layers "B.Cu") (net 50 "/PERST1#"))
  (pad "67" smd rect (at -7.25 -0.04 180) (size 0.35 1.7) (layers "F.Cu") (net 4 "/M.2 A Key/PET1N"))
  (pad "68" smd rect (at -7.5 -0.29 180) (size 0.35 2.2) (layers "B.Cu") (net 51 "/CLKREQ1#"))
  (pad "69" smd rect (at -7.75 -0.04 180) (size 0.35 1.7) (layers "F.Cu") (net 3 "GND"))
  (pad "70" smd rect (at -8 -0.29 180) (size 0.35 2.2) (layers "B.Cu") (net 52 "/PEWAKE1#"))
  (pad "71" smd rect (at -8.25 -0.04 180) (size 0.35 1.7) (layers "F.Cu") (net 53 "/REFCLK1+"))
  (pad "72" smd rect (at -8.5 -0.29 180) (size 0.35 2.2) (layers "B.Cu") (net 11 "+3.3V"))
  (pad "73" smd rect (at -8.75 -0.04 180) (size 0.35 1.7) (layers "F.Cu") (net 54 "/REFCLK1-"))
  (pad "74" smd rect (at -9 -0.29 180) (size 0.35 2.2) (layers "B.Cu") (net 11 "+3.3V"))
  (pad "75" smd rect (at -9.25 -0.04 180) (size 0.35 1.7) (layers "F.Cu") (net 3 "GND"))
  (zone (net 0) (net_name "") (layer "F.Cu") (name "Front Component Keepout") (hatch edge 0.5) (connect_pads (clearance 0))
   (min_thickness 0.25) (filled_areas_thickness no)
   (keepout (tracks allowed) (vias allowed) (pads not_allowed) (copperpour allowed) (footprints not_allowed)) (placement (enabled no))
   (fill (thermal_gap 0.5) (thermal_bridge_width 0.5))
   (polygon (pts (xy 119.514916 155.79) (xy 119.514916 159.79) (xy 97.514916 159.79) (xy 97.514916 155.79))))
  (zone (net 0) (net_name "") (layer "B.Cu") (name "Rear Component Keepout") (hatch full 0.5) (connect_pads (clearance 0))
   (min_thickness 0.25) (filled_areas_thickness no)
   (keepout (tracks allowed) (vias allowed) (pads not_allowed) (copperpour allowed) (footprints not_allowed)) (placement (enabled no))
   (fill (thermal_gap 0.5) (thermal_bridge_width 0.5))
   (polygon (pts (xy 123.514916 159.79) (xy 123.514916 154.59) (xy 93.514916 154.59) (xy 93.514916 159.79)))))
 (gr_line (start 97.514916 79.79) (end 97.514916 155.79) (stroke (width 0.1) (type default)) (layer "Edge.Cuts"))
 (gr_line (start 119.514916 155.79) (end 119.514916 79.79) (stroke (width 0.1) (type default)) (layer "Edge.Cuts"))
 (gr_line (start 119.514916 79.79) (end 97.514916 79.79) (stroke (width 0.1) (type solid)) (layer "Edge.Cuts"))
 (via (at 109.014916 156.709) (size 0.6) (drill 0.3) (layers "F.Cu" "B.Cu") (free yes) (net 3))
 (via (at 113.514916 156.709) (size 0.6) (drill 0.3) (layers "F.Cu" "B.Cu") (free yes) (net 3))
 (via (at 110.514916 156.709) (size 0.6) (drill 0.3) (layers "F.Cu" "B.Cu") (free yes) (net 3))
 (via (at 112.014916 156.709) (size 0.6) (drill 0.3) (layers "F.Cu" "B.Cu") (free yes) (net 3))
 (segment (start 101.739916 157.339999) (end 101.739916 155.834001) (width 0.2) (layer "F.Cu") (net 1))
 (segment (start 101.739916 155.834001) (end 101.864916 155.709001) (width 0.2) (layer "F.Cu") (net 1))
 (segment (start 101.764916 158.64) (end 101.764916 157.364999) (width 0.2) (layer "F.Cu") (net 1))
 (segment (start 101.764916 157.364999) (end 101.739916 157.339999) (width 0.2) (layer "F.Cu") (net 1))
 (segment (start 101.864916 155.709001) (end 101.864916 155.364) (width 0.2) (layer "F.Cu") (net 1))
 (segment (start 101.264916 157.364999) (end 101.289916 157.339999) (width 0.2) (layer "F.Cu") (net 4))
 (segment (start 101.264916 158.64) (end 101.264916 157.364999) (width 0.2) (layer "F.Cu") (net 4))
 (segment (start 101.289916 155.834001) (end 101.164916 155.709001) (width 0.2) (layer "F.Cu") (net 4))
 (segment (start 101.164916 155.709001) (end 101.164916 155.364) (width 0.2) (layer "F.Cu") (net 4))
 (segment (start 101.289916 157.339999) (end 101.289916 155.834001) (width 0.2) (layer "F.Cu") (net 4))
 (segment (start 107.864916 155.709001) (end 107.864916 155.364) (width 0.2) (layer "F.Cu") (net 6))
 (segment (start 107.739916 155.834001) (end 107.864916 155.709001) (width 0.2) (layer "F.Cu") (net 6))
 (segment (start 107.739916 157.339999) (end 107.739916 155.834001) (width 0.2) (layer "F.Cu") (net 6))
 (segment (start 107.764916 158.64) (end 107.764916 157.364999) (width 0.2) (layer "F.Cu") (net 6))
 (segment (start 107.764916 157.364999) (end 107.739916 157.339999) (width 0.2) (layer "F.Cu") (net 6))
 (segment (start 107.264916 157.364999) (end 107.289916 157.339999) (width 0.2) (layer "F.Cu") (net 8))
 (segment (start 107.289916 157.339999) (end 107.289916 155.834001) (width 0.2) (layer "F.Cu") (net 8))
 (segment (start 107.164916 155.709001) (end 107.164916 155.364) (width 0.2) (layer "F.Cu") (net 8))
 (segment (start 107.289916 155.834001) (end 107.164916 155.709001) (width 0.2) (layer "F.Cu") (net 8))
 (segment (start 107.264916 158.64) (end 107.264916 157.364999) (width 0.2) (layer "F.Cu") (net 8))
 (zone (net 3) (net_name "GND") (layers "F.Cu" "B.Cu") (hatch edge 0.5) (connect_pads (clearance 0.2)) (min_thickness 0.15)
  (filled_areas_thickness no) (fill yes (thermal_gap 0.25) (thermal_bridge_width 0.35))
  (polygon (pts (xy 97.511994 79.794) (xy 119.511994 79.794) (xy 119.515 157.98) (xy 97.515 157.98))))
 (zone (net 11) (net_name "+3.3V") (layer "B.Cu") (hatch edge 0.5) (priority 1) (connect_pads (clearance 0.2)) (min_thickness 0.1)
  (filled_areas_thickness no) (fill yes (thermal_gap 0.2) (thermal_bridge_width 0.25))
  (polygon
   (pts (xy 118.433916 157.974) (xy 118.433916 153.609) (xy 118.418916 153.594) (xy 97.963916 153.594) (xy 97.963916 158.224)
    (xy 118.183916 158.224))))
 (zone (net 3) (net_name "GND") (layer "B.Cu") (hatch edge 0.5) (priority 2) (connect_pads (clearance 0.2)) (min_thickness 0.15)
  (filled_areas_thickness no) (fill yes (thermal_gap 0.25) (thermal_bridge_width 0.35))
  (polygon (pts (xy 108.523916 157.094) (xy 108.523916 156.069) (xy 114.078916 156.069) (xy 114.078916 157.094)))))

